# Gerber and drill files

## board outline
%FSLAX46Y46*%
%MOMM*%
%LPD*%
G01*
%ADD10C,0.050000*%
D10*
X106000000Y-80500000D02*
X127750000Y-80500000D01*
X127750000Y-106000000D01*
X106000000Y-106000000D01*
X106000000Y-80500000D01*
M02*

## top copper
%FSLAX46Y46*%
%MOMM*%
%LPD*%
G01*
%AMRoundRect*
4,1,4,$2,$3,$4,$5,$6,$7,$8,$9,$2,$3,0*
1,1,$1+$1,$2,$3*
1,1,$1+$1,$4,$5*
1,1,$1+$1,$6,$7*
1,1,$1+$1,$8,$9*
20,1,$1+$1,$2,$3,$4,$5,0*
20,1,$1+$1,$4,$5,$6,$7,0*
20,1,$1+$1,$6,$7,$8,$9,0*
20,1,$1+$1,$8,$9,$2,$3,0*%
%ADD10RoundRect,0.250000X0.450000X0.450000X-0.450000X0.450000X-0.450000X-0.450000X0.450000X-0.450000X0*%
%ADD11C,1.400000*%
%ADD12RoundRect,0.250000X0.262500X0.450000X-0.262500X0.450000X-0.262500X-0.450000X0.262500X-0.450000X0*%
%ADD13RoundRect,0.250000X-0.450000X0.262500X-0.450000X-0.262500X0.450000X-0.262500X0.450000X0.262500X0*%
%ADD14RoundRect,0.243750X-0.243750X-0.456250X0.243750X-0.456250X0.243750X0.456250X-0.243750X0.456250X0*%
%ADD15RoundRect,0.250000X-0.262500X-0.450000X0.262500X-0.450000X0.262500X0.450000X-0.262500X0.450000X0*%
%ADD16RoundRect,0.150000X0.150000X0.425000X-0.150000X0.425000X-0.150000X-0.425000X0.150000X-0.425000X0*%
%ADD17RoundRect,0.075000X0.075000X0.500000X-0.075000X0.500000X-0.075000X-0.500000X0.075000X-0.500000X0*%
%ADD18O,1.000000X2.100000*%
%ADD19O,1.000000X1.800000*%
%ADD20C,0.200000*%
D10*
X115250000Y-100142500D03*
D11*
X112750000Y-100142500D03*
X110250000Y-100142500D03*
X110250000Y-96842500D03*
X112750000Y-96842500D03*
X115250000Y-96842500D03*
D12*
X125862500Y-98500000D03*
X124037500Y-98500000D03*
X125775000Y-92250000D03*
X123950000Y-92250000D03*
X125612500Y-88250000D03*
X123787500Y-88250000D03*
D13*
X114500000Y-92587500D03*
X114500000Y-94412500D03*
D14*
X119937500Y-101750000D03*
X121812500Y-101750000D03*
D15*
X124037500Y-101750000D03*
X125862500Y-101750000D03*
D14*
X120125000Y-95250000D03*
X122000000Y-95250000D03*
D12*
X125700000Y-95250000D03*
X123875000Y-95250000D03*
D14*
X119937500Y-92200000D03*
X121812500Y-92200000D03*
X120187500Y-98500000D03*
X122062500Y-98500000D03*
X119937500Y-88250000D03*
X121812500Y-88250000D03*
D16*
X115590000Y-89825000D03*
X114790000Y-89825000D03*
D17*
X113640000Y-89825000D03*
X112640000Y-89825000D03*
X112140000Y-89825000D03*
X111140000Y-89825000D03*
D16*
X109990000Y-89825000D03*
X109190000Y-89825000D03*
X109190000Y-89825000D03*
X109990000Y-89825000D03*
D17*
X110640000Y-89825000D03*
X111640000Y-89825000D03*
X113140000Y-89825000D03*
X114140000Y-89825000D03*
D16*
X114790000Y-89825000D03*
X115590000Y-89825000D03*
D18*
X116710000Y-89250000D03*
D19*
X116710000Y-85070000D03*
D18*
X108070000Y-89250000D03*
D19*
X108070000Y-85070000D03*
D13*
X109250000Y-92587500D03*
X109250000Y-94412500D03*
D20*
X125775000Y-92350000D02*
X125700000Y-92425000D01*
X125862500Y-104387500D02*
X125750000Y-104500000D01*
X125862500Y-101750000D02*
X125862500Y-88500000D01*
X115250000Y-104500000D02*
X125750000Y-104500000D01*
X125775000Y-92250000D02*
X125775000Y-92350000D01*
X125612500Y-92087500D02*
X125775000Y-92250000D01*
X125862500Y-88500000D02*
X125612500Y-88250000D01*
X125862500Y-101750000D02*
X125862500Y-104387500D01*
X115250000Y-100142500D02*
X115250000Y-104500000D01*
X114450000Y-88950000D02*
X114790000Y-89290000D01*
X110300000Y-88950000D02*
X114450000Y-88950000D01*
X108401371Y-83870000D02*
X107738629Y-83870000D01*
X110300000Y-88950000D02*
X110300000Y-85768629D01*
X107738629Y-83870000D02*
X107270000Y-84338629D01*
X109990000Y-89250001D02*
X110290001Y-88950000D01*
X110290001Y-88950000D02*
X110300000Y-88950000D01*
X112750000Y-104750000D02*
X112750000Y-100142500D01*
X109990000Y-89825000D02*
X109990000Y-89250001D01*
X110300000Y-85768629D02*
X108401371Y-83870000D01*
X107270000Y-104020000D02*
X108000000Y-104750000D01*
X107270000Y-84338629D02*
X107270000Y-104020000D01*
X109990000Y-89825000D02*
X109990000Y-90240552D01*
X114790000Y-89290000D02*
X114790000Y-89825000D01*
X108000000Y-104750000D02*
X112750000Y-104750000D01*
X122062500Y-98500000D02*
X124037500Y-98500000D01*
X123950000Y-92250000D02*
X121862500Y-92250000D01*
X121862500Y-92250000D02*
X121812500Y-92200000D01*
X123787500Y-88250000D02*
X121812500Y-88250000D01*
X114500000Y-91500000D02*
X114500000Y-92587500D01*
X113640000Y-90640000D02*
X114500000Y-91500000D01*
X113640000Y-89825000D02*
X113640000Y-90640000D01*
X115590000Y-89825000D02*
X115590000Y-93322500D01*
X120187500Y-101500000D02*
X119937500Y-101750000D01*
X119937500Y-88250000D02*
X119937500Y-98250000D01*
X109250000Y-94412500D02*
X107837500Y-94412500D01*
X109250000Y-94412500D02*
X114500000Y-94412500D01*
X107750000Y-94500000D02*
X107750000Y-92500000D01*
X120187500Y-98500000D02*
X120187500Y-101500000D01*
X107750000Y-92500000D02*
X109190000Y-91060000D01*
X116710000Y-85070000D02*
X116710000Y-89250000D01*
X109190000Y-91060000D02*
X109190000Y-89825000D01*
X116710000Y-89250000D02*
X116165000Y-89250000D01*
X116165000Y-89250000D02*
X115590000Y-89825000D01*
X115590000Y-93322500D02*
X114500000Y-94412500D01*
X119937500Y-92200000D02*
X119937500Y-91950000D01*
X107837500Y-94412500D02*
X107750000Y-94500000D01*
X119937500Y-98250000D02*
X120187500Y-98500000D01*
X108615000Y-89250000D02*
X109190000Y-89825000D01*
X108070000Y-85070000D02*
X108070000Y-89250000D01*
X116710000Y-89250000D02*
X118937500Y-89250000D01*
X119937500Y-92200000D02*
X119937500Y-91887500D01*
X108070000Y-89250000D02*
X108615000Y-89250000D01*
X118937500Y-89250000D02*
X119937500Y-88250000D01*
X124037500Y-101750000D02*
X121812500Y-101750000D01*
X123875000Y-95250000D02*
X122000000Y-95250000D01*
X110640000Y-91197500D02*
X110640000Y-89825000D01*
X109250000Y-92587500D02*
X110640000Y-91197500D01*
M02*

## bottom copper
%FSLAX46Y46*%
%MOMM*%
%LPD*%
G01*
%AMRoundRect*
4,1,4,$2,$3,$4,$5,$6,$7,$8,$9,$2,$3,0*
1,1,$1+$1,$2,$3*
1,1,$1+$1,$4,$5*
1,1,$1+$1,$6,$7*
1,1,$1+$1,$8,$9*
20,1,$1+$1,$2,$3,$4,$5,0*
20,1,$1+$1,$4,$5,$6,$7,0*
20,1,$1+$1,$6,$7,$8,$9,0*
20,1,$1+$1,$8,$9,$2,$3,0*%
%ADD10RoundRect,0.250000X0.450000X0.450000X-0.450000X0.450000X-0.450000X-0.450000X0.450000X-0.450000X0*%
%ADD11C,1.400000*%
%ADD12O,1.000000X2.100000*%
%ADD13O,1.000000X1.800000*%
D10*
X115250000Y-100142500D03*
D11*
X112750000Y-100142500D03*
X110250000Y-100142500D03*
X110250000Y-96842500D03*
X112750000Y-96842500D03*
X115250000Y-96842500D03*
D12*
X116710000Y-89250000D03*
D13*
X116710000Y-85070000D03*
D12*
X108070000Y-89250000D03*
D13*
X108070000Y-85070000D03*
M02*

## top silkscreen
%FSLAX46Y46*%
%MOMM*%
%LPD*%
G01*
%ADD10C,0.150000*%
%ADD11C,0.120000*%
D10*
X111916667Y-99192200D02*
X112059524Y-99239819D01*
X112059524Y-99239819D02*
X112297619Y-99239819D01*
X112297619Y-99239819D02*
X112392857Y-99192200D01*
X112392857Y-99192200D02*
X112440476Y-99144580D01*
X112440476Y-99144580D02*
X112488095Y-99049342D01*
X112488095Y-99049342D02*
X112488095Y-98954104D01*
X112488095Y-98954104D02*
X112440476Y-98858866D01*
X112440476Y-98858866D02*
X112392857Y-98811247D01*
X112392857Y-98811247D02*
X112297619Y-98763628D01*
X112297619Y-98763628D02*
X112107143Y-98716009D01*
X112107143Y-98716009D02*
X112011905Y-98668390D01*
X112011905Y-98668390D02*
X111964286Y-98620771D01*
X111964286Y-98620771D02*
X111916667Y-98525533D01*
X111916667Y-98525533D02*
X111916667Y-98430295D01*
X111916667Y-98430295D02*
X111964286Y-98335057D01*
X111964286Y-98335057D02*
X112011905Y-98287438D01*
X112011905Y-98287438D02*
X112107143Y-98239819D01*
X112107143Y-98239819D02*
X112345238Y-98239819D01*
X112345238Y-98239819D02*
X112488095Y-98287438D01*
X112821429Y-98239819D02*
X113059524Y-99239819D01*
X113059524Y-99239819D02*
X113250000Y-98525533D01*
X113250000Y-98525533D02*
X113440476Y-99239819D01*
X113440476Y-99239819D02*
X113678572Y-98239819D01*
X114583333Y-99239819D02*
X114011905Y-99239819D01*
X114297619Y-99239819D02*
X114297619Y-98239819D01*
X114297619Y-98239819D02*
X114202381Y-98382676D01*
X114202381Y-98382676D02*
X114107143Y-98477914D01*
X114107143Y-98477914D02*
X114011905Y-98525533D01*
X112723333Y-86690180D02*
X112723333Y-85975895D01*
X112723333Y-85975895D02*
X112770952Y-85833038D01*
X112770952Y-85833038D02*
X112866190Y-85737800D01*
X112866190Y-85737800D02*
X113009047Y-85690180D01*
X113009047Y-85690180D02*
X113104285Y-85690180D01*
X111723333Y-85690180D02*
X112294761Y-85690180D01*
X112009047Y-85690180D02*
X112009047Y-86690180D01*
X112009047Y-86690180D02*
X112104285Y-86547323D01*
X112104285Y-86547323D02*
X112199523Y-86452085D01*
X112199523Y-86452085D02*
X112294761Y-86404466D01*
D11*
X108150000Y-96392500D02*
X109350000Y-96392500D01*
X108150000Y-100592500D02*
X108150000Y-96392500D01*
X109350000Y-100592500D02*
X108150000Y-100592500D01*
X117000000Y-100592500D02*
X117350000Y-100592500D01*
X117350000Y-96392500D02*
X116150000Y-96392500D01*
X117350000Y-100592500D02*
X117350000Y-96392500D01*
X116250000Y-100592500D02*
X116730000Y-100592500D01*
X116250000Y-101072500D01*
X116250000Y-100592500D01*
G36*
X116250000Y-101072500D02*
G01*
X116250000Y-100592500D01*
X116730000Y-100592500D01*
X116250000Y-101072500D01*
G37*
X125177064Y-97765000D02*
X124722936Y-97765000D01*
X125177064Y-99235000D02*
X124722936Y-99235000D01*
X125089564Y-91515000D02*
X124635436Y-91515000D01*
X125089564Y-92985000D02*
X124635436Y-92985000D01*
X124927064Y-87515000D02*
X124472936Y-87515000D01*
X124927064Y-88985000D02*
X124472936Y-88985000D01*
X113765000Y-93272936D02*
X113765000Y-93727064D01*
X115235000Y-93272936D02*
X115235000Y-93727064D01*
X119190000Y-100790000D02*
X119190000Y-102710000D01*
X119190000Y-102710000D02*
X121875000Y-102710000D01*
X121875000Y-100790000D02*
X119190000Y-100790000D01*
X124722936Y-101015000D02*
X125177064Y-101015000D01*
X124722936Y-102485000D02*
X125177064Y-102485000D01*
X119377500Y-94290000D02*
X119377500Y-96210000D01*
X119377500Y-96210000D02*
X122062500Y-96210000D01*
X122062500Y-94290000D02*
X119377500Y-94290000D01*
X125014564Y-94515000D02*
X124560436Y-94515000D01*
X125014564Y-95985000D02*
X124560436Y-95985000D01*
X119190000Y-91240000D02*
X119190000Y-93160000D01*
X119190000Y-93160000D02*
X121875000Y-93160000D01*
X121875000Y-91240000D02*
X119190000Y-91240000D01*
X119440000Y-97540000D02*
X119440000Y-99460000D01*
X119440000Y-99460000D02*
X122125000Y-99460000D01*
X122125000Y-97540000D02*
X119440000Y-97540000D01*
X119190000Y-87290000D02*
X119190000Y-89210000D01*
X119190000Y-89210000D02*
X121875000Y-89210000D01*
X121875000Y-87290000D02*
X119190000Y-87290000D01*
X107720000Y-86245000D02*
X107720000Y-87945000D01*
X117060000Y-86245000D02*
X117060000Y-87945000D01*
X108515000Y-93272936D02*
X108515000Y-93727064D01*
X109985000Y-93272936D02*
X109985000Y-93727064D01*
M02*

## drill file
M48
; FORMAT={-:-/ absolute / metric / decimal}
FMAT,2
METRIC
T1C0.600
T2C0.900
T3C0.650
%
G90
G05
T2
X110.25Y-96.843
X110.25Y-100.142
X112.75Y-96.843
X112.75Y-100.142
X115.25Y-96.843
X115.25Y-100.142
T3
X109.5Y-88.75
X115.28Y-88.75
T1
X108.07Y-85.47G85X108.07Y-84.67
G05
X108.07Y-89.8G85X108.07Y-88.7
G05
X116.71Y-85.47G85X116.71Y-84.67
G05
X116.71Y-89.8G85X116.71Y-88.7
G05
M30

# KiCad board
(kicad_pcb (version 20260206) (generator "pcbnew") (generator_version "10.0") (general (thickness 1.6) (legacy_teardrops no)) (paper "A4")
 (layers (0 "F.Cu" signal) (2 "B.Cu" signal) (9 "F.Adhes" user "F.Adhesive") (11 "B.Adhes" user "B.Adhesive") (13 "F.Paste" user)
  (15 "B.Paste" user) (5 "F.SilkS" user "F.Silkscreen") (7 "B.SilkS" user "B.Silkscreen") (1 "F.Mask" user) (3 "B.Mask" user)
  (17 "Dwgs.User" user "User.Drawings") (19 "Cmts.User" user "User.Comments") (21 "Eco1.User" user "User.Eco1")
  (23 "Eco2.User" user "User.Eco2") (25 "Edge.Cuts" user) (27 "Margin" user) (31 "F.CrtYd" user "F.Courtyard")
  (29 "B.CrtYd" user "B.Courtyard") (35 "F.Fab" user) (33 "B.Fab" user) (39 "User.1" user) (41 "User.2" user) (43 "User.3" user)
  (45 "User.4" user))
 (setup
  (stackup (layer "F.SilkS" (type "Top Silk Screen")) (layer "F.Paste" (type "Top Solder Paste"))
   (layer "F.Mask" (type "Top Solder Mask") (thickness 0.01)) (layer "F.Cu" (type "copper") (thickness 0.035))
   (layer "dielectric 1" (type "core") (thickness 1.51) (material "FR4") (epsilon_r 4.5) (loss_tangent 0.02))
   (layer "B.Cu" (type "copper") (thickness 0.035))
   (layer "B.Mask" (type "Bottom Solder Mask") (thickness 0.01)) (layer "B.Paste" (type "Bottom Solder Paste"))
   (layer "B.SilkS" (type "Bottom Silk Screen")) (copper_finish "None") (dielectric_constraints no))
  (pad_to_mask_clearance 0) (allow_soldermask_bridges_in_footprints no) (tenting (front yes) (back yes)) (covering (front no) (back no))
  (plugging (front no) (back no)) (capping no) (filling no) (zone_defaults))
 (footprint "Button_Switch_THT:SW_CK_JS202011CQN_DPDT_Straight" (layer "F.Cu") (at 115.25 100.1425 180)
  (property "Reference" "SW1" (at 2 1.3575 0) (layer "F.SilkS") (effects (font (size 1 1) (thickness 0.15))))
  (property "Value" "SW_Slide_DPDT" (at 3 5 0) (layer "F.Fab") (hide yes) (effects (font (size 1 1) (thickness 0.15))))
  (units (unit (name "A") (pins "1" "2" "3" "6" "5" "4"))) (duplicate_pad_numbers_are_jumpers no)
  (fp_line (start 7.1 3.75) (end 5.9 3.75) (stroke (width 0.12) (type solid)) (layer "F.SilkS"))
  (fp_line (start 7.1 -0.45) (end 7.1 3.75) (stroke (width 0.12) (type solid)) (layer "F.SilkS"))
  (fp_line (start 5.9 -0.45) (end 7.1 -0.45) (stroke (width 0.12) (type solid)) (layer "F.SilkS"))
  (fp_line (start -1.75 -0.45) (end -2.1 -0.45) (stroke (width 0.12) (type solid)) (layer "F.SilkS"))
  (fp_line (start -2.1 3.75) (end -0.9 3.75) (stroke (width 0.12) (type solid)) (layer "F.SilkS"))
  (fp_line (start -2.1 -0.45) (end -2.1 3.75) (stroke (width 0.12) (type solid)) (layer "F.SilkS"))
  (fp_poly (pts (xy -1 -0.45) (xy -1.48 -0.45) (xy -1 -0.93) (xy -1 -0.45)) (stroke (width 0.12) (type solid)) (fill yes) (layer "F.SilkS"))
  (pad "1" thru_hole roundrect (at 0 0 180) (size 1.4 1.4) (drill 0.9) (layers "*.Cu" "*.Mask") (remove_unused_layers no)
   (roundrect_rratio 0.1785714286) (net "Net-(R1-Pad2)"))
  (pad "2" thru_hole circle (at 2.5 0 180) (size 1.4 1.4) (drill 0.9) (layers "*.Cu" "*.Mask") (remove_unused_layers no)
   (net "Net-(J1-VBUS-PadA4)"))
  (pad "3" thru_hole circle (at 5 0 180) (size 1.4 1.4) (drill 0.9) (layers "*.Cu" "*.Mask") (remove_unused_layers no)
   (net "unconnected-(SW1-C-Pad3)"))
  (pad "4" thru_hole circle (at 5 3.3 180) (size 1.4 1.4) (drill 0.9) (layers "*.Cu" "*.Mask") (remove_unused_layers no)
   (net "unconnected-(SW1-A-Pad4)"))
  (pad "5" thru_hole circle (at 2.5 3.3 180) (size 1.4 1.4) (drill 0.9) (layers "*.Cu" "*.Mask") (remove_unused_layers no)
   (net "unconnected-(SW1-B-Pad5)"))
  (pad "6" thru_hole circle (at 0 3.3 180) (size 1.4 1.4) (drill 0.9) (layers "*.Cu" "*.Mask") (remove_unused_layers no)
   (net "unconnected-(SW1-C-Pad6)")))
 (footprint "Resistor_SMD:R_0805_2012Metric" (layer "F.Cu") (at 124.95 98.5 180)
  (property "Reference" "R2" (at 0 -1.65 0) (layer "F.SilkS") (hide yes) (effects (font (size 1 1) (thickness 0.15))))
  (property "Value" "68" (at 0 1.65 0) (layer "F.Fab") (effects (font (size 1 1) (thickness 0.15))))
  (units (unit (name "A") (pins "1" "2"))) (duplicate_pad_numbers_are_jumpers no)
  (fp_line (start -0.227064 0.735) (end 0.227064 0.735) (stroke (width 0.12) (type solid)) (layer "F.SilkS"))
  (fp_line (start -0.227064 -0.735) (end 0.227064 -0.735) (stroke (width 0.12) (type solid)) (layer "F.SilkS"))
  (pad "1" smd roundrect (at -0.9125 0 180) (size 1.025 1.4) (layers "F.Cu" "F.Mask" "F.Paste") (roundrect_rratio 0.243902)
   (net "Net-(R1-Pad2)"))
  (pad "2" smd roundrect (at 0.9125 0 180) (size 1.025 1.4) (layers "F.Cu" "F.Mask" "F.Paste") (roundrect_rratio 0.243902)
   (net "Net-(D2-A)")))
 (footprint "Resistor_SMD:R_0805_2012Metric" (layer "F.Cu") (at 124.8625 92.25 180)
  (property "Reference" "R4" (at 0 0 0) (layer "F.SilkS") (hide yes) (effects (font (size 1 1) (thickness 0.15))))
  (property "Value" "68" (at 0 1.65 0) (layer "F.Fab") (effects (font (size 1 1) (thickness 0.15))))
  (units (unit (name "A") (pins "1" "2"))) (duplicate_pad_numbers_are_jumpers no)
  (fp_line (start -0.227064 0.735) (end 0.227064 0.735) (stroke (width 0.12) (type solid)) (layer "F.SilkS"))
  (fp_line (start -0.227064 -0.735) (end 0.227064 -0.735) (stroke (width 0.12) (type solid)) (layer "F.SilkS"))
  (pad "1" smd roundrect (at -0.9125 0 180) (size 1.025 1.4) (layers "F.Cu" "F.Mask" "F.Paste") (roundrect_rratio 0.243902)
   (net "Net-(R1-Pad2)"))
  (pad "2" smd roundrect (at 0.9125 0 180) (size 1.025 1.4) (layers "F.Cu" "F.Mask" "F.Paste") (roundrect_rratio 0.243902)
   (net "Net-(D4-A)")))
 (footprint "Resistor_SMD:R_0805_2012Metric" (layer "F.Cu") (at 124.7 88.25 180)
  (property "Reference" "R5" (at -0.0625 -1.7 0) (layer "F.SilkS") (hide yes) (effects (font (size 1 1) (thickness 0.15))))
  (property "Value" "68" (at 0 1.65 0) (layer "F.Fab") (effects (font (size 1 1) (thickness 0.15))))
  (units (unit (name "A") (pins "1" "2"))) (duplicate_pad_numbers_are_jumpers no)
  (fp_line (start -0.227064 0.735) (end 0.227064 0.735) (stroke (width 0.12) (type solid)) (layer "F.SilkS"))
  (fp_line (start -0.227064 -0.735) (end 0.227064 -0.735) (stroke (width 0.12) (type solid)) (layer "F.SilkS"))
  (pad "1" smd roundrect (at -0.9125 0 180) (size 1.025 1.4) (layers "F.Cu" "F.Mask" "F.Paste") (roundrect_rratio 0.243902)
   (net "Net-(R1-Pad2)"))
  (pad "2" smd roundrect (at 0.9125 0 180) (size 1.025 1.4) (layers "F.Cu" "F.Mask" "F.Paste") (roundrect_rratio 0.243902)
   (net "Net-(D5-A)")))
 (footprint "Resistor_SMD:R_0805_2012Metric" (layer "F.Cu") (at 114.5 93.5 -90)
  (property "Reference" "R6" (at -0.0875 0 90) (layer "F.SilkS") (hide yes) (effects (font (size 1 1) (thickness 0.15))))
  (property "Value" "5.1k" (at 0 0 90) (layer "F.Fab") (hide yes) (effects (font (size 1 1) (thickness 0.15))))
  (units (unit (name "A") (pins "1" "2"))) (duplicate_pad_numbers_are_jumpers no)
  (fp_line (start -0.227064 0.735) (end 0.227064 0.735) (stroke (width 0.12) (type solid)) (layer "F.SilkS"))
  (fp_line (start -0.227064 -0.735) (end 0.227064 -0.735) (stroke (width 0.12) (type solid)) (layer "F.SilkS"))
  (pad "1" smd roundrect (at -0.9125 0 270) (size 1.025 1.4) (layers "F.Cu" "F.Mask" "F.Paste") (roundrect_rratio 0.243902)
   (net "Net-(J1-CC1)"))
  (pad "2" smd roundrect (at 0.9125 0 270) (size 1.025 1.4) (layers "F.Cu" "F.Mask" "F.Paste") (roundrect_rratio 0.243902)
   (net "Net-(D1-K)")))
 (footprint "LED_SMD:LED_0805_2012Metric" (layer "F.Cu") (at 120.875 101.75)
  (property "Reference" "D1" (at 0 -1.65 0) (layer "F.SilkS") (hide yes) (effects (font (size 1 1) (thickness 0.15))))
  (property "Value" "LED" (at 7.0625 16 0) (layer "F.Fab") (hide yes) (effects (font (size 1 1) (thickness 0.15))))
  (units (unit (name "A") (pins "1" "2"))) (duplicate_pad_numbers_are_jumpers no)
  (fp_line (start -1.685 -0.96) (end -1.685 0.96) (stroke (width 0.12) (type solid)) (layer "F.SilkS"))
  (fp_line (start -1.685 0.96) (end 1 0.96) (stroke (width 0.12) (type solid)) (layer "F.SilkS"))
  (fp_line (start 1 -0.96) (end -1.685 -0.96) (stroke (width 0.12) (type solid)) (layer "F.SilkS"))
  (pad "1" smd roundrect (at -0.9375 0) (size 0.975 1.4) (layers "F.Cu" "F.Mask" "F.Paste") (roundrect_rratio 0.25) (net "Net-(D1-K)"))
  (pad "2" smd roundrect (at 0.9375 0) (size 0.975 1.4) (layers "F.Cu" "F.Mask" "F.Paste") (roundrect_rratio 0.25) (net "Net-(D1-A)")))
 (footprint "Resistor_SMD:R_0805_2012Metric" (layer "F.Cu") (at 124.95 101.75)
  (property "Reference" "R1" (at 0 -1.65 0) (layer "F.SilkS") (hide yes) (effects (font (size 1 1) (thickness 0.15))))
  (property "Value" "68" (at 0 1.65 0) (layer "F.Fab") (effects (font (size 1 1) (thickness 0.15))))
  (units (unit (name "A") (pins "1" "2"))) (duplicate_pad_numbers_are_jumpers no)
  (fp_line (start -0.227064 -0.735) (end 0.227064 -0.735) (stroke (width 0.12) (type solid)) (layer "F.SilkS"))
  (fp_line (start -0.227064 0.735) (end 0.227064 0.735) (stroke (width 0.12) (type solid)) (layer "F.SilkS"))
  (pad "1" smd roundrect (at -0.9125 0) (size 1.025 1.4) (layers "F.Cu" "F.Mask" "F.Paste") (roundrect_rratio 0.243902) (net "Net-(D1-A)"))
  (pad "2" smd roundrect (at 0.9125 0) (size 1.025 1.4) (layers "F.Cu" "F.Mask" "F.Paste") (roundrect_rratio 0.243902) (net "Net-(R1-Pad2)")))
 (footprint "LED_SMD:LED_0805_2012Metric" (layer "F.Cu") (at 121.0625 95.25)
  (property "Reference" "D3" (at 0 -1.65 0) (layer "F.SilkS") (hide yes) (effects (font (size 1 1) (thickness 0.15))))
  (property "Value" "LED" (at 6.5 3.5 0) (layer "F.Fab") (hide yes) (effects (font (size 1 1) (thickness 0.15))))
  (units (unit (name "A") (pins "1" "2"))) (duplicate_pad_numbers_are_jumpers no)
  (fp_line (start -1.685 -0.96) (end -1.685 0.96) (stroke (width 0.12) (type solid)) (layer "F.SilkS"))
  (fp_line (start -1.685 0.96) (end 1 0.96) (stroke (width 0.12) (type solid)) (layer "F.SilkS"))
  (fp_line (start 1 -0.96) (end -1.685 -0.96) (stroke (width 0.12) (type solid)) (layer "F.SilkS"))
  (pad "1" smd roundrect (at -0.9375 0) (size 0.975 1.4) (layers "F.Cu" "F.Mask" "F.Paste") (roundrect_rratio 0.25) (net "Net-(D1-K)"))
  (pad "2" smd roundrect (at 0.9375 0) (size 0.975 1.4) (layers "F.Cu" "F.Mask" "F.Paste") (roundrect_rratio 0.25) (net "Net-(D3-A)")))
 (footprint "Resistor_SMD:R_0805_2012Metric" (layer "F.Cu") (at 124.7875 95.25 180)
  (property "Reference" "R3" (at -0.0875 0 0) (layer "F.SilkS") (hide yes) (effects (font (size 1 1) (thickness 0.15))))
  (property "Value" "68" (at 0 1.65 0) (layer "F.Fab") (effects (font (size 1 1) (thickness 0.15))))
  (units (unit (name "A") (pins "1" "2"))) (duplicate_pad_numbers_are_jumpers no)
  (fp_line (start -0.227064 0.735) (end 0.227064 0.735) (stroke (width 0.12) (type solid)) (layer "F.SilkS"))
  (fp_line (start -0.227064 -0.735) (end 0.227064 -0.735) (stroke (width 0.12) (type solid)) (layer "F.SilkS"))
  (pad "1" smd roundrect (at -0.9125 0 180) (size 1.025 1.4) (layers "F.Cu" "F.Mask" "F.Paste") (roundrect_rratio 0.243902)
   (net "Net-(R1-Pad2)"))
  (pad "2" smd roundrect (at 0.9125 0 180) (size 1.025 1.4) (layers "F.Cu" "F.Mask" "F.Paste") (roundrect_rratio 0.243902)
   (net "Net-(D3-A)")))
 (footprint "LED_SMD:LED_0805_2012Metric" (layer "F.Cu") (at 120.875 92.2)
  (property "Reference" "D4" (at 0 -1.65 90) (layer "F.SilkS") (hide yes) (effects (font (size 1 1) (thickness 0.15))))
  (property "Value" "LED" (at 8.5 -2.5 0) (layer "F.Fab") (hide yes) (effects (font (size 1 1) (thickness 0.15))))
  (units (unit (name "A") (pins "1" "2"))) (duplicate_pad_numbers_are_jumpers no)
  (fp_line (start -1.685 -0.96) (end -1.685 0.96) (stroke (width 0.12) (type solid)) (layer "F.SilkS"))
  (fp_line (start -1.685 0.96) (end 1 0.96) (stroke (width 0.12) (type solid)) (layer "F.SilkS"))
  (fp_line (start 1 -0.96) (end -1.685 -0.96) (stroke (width 0.12) (type solid)) (layer "F.SilkS"))
  (pad "1" smd roundrect (at -0.9375 0) (size 0.975 1.4) (layers "F.Cu" "F.Mask" "F.Paste") (roundrect_rratio 0.25) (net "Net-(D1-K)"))
  (pad "2" smd roundrect (at 0.9375 0) (size 0.975 1.4) (layers "F.Cu" "F.Mask" "F.Paste") (roundrect_rratio 0.25) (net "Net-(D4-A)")))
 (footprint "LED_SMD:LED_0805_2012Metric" (layer "F.Cu") (at 121.125 98.5)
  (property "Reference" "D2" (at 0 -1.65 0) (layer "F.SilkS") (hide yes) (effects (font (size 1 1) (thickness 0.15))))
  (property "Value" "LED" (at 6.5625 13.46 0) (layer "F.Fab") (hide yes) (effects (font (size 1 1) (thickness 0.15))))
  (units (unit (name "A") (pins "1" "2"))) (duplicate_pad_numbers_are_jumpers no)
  (fp_line (start -1.685 -0.96) (end -1.685 0.96) (stroke (width 0.12) (type solid)) (layer "F.SilkS"))
  (fp_line (start -1.685 0.96) (end 1 0.96) (stroke (width 0.12) (type solid)) (layer "F.SilkS"))
  (fp_line (start 1 -0.96) (end -1.685 -0.96) (stroke (width 0.12) (type solid)) (layer "F.SilkS"))
  (pad "1" smd roundrect (at -0.9375 0) (size 0.975 1.4) (layers "F.Cu" "F.Mask" "F.Paste") (roundrect_rratio 0.25) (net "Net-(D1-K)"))
  (pad "2" smd roundrect (at 0.9375 0) (size 0.975 1.4) (layers "F.Cu" "F.Mask" "F.Paste") (roundrect_rratio 0.25) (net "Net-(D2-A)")))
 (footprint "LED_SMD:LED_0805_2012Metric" (layer "F.Cu") (at 120.875 88.25)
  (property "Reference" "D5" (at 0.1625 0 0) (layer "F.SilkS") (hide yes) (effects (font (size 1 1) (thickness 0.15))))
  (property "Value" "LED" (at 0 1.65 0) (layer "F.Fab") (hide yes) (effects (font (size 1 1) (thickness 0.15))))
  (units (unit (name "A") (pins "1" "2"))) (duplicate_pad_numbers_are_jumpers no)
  (fp_line (start -1.685 -0.96) (end -1.685 0.96) (stroke (width 0.12) (type solid)) (layer "F.SilkS"))
  (fp_line (start -1.685 0.96) (end 1 0.96) (stroke (width 0.12) (type solid)) (layer "F.SilkS"))
  (fp_line (start 1 -0.96) (end -1.685 -0.96) (stroke (width 0.12) (type solid)) (layer "F.SilkS"))
  (pad "1" smd roundrect (at -0.9375 0) (size 0.975 1.4) (layers "F.Cu" "F.Mask" "F.Paste") (roundrect_rratio 0.25) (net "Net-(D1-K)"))
  (pad "2" smd roundrect (at 0.9375 0) (size 0.975 1.4) (layers "F.Cu" "F.Mask" "F.Paste") (roundrect_rratio 0.25) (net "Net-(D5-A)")))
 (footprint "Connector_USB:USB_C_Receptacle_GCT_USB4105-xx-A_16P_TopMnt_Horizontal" (layer "F.Cu") (at 112.39 86.145 180)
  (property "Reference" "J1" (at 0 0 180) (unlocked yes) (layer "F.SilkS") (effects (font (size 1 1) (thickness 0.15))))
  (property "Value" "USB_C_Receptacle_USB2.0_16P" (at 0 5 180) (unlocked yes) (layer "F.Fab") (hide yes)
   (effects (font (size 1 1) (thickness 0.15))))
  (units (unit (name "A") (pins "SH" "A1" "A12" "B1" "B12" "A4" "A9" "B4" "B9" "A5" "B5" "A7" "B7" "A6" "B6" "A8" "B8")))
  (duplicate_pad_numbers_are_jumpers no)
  (fp_line (start 4.67 -0.1) (end 4.67 -1.8) (stroke (width 0.12) (type solid)) (layer "F.SilkS"))
  (fp_line (start -4.67 -0.1) (end -4.67 -1.8) (stroke (width 0.12) (type solid)) (layer "F.SilkS"))
  (pad "" np_thru_hole circle (at -2.89 -2.605 180) (size 0.65 0.65) (drill 0.65) (layers "*.Cu" "*.Mask"))
  (pad "" np_thru_hole circle (at 2.89 -2.605 180) (size 0.65 0.65) (drill 0.65) (layers "*.Cu" "*.Mask"))
  (pad "A1" smd roundrect (at -3.2 -3.68 180) (size 0.6 1.15) (layers "F.Cu" "F.Mask" "F.Paste") (roundrect_rratio 0.25) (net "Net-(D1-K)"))
  (pad "A4" smd roundrect (at -2.4 -3.68 180) (size 0.6 1.15) (layers "F.Cu" "F.Mask" "F.Paste") (roundrect_rratio 0.25)
   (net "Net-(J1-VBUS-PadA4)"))
  (pad "A5" smd roundrect (at -1.25 -3.68 180) (size 0.3 1.15) (layers "F.Cu" "F.Mask" "F.Paste") (roundrect_rratio 0.25)
   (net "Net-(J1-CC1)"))
  (pad "A6" smd roundrect (at -0.25 -3.68 180) (size 0.3 1.15) (layers "F.Cu" "F.Mask" "F.Paste") (roundrect_rratio 0.25)
   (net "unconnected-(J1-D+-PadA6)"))
  (pad "A7" smd roundrect (at 0.25 -3.68 180) (size 0.3 1.15) (layers "F.Cu" "F.Mask" "F.Paste") (roundrect_rratio 0.25)
   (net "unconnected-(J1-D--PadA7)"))
  (pad "A8" smd roundrect (at 1.25 -3.68 180) (size 0.3 1.15) (layers "F.Cu" "F.Mask" "F.Paste") (roundrect_rratio 0.25)
   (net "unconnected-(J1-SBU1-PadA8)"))
  (pad "A9" smd roundrect (at 2.4 -3.68 180) (size 0.6 1.15) (layers "F.Cu" "F.Mask" "F.Paste") (roundrect_rratio 0.25)
   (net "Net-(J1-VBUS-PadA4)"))
  (pad "A12" smd roundrect (at 3.2 -3.68 180) (size 0.6 1.15) (layers "F.Cu" "F.Mask" "F.Paste") (roundrect_rratio 0.25) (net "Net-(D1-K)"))
  (pad "B1" smd roundrect (at 3.2 -3.68 180) (size 0.6 1.15) (layers "F.Cu" "F.Mask" "F.Paste") (roundrect_rratio 0.25) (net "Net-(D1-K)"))
  (pad "B4" smd roundrect (at 2.4 -3.68 180) (size 0.6 1.15) (layers "F.Cu" "F.Mask" "F.Paste") (roundrect_rratio 0.25)
   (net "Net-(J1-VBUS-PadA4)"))
  (pad "B5" smd roundrect (at 1.75 -3.68 180) (size 0.3 1.15) (layers "F.Cu" "F.Mask" "F.Paste") (roundrect_rratio 0.25)
   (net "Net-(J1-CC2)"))
  (pad "B6" smd roundrect (at 0.75 -3.68 180) (size 0.3 1.15) (layers "F.Cu" "F.Mask" "F.Paste") (roundrect_rratio 0.25)
   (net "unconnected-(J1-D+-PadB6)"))
  (pad "B7" smd roundrect (at -0.75 -3.68 180) (size 0.3 1.15) (layers "F.Cu" "F.Mask" "F.Paste") (roundrect_rratio 0.25)
   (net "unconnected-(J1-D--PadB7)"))
  (pad "B8" smd roundrect (at -1.75 -3.68 180) (size 0.3 1.15) (layers "F.Cu" "F.Mask" "F.Paste") (roundrect_rratio 0.25)
   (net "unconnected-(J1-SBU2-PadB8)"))
  (pad "B9" smd roundrect (at -2.4 -3.68 180) (size 0.6 1.15) (layers "F.Cu" "F.Mask" "F.Paste") (roundrect_rratio 0.25)
   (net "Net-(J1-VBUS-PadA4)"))
  (pad "B12" smd roundrect (at -3.2 -3.68 180) (size 0.6 1.15) (layers "F.Cu" "F.Mask" "F.Paste") (roundrect_rratio 0.25) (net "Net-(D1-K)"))
  (pad "SH" thru_hole oval (at -4.32 -3.105 180) (size 1 2.1) (drill oval 0.6 1.7) (layers "*.Cu" "*.Mask" "F.Paste")
   (remove_unused_layers no) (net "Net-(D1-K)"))
  (pad "SH" thru_hole oval (at -4.32 1.075 180) (size 1 1.8) (drill oval 0.6 1.4) (layers "*.Cu" "*.Mask" "F.Paste")
   (remove_unused_layers no) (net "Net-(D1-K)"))
  (pad "SH" thru_hole oval (at 4.32 -3.105 180) (size 1 2.1) (drill oval 0.6 1.7) (layers "*.Cu" "*.Mask" "F.Paste")
   (remove_unused_layers no) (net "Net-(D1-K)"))
  (pad "SH" thru_hole oval (at 4.32 1.075 180) (size 1 1.8) (drill oval 0.6 1.4) (layers "*.Cu" "*.Mask" "F.Paste")
   (remove_unused_layers no) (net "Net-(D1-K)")))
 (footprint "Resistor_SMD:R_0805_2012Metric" (layer "F.Cu") (at 109.25 93.5 -90)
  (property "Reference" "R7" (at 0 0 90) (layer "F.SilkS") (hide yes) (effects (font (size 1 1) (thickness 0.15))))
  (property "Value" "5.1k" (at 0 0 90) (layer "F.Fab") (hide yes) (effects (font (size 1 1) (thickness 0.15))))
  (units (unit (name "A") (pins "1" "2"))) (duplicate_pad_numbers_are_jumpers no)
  (fp_line (start -0.227064 0.735) (end 0.227064 0.735) (stroke (width 0.12) (type solid)) (layer "F.SilkS"))
  (fp_line (start -0.227064 -0.735) (end 0.227064 -0.735) (stroke (width 0.12) (type solid)) (layer "F.SilkS"))
  (pad "1" smd roundrect (at -0.9125 0 270) (size 1.025 1.4) (layers "F.Cu" "F.Mask" "F.Paste") (roundrect_rratio 0.243902)
   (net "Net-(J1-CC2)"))
  (pad "2" smd roundrect (at 0.9125 0 270) (size 1.025 1.4) (layers "F.Cu" "F.Mask" "F.Paste") (roundrect_rratio 0.243902)
   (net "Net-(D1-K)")))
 (gr_rect (start 106 80.5) (end 127.75 106) (stroke (width 0.05) (type default)) (fill no) (layer "Edge.Cuts"))
 (segment (start 125.775 92.35) (end 125.7 92.425) (width 0.2) (layer "F.Cu") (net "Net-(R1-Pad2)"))
 (segment (start 125.8625 104.3875) (end 125.75 104.5) (width 0.2) (layer "F.Cu") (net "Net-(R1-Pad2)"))
 (segment (start 125.8625 101.75) (end 125.8625 88.5) (width 0.2) (layer "F.Cu") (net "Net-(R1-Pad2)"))
 (segment (start 115.25 104.5) (end 125.75 104.5) (width 0.2) (layer "F.Cu") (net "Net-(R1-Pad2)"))
 (segment (start 125.775 92.25) (end 125.775 92.35) (width 0.2) (layer "F.Cu") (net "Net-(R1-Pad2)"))
 (segment (start 125.6125 92.0875) (end 125.775 92.25) (width 0.2) (layer "F.Cu") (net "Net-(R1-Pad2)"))
 (segment (start 125.8625 88.5) (end 125.6125 88.25) (width 0.2) (layer "F.Cu") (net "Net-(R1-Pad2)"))
 (segment (start 125.8625 101.75) (end 125.8625 104.3875) (width 0.2) (layer "F.Cu") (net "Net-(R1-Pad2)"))
 (segment (start 115.25 100.1425) (end 115.25 104.5) (width 0.2) (layer "F.Cu") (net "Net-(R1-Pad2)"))
 (segment (start 114.45 88.95) (end 114.79 89.29) (width 0.2) (layer "F.Cu") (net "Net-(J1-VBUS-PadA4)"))
 (segment (start 110.3 88.95) (end 114.45 88.95) (width 0.2) (layer "F.Cu") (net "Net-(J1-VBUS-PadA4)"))
 (segment (start 108.401371 83.87) (end 107.738629 83.87) (width 0.2) (layer "F.Cu") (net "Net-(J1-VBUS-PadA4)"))
 (segment (start 110.3 88.95) (end 110.3 85.768629) (width 0.2) (layer "F.Cu") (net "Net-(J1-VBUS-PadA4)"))
 (segment (start 107.738629 83.87) (end 107.27 84.338629) (width 0.2) (layer "F.Cu") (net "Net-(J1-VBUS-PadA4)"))
 (segment (start 109.99 89.250001) (end 110.290001 88.95) (width 0.2) (layer "F.Cu") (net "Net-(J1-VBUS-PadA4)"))
 (segment (start 110.290001 88.95) (end 110.3 88.95) (width 0.2) (layer "F.Cu") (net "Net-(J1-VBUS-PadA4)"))
 (segment (start 112.75 104.75) (end 112.75 100.1425) (width 0.2) (layer "F.Cu") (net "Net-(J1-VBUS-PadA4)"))
 (segment (start 109.99 89.825) (end 109.99 89.250001) (width 0.2) (layer "F.Cu") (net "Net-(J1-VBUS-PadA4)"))
 (segment (start 110.3 85.768629) (end 108.401371 83.87) (width 0.2) (layer "F.Cu") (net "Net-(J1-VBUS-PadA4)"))
 (segment (start 107.27 104.02) (end 108 104.75) (width 0.2) (layer "F.Cu") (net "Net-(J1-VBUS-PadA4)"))
 (segment (start 107.27 84.338629) (end 107.27 104.02) (width 0.2) (layer "F.Cu") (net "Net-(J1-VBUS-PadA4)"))
 (segment (start 109.99 89.825) (end 109.99 90.240552) (width 0.2) (layer "F.Cu") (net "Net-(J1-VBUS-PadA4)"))
 (segment (start 114.79 89.29) (end 114.79 89.825) (width 0.2) (layer "F.Cu") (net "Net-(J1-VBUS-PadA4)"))
 (segment (start 108 104.75) (end 112.75 104.75) (width 0.2) (layer "F.Cu") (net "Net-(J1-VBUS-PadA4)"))
 (segment (start 122.0625 98.5) (end 124.0375 98.5) (width 0.2) (layer "F.Cu") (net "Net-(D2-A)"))
 (segment (start 123.95 92.25) (end 121.8625 92.25) (width 0.2) (layer "F.Cu") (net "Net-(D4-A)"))
 (segment (start 121.8625 92.25) (end 121.8125 92.2) (width 0.2) (layer "F.Cu") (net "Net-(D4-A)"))
 (segment (start 123.7875 88.25) (end 121.8125 88.25) (width 0.2) (layer "F.Cu") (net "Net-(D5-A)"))
 (segment (start 114.5 91.5) (end 114.5 92.5875) (width 0.2) (layer "F.Cu") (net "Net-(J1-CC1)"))
 (segment (start 113.64 90.64) (end 114.5 91.5) (width 0.2) (layer "F.Cu") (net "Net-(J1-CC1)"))
 (segment (start 113.64 89.825) (end 113.64 90.64) (width 0.2) (layer "F.Cu") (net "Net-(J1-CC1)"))
 (segment (start 115.59 89.825) (end 115.59 93.3225) (width 0.2) (layer "F.Cu") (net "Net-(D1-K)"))
 (segment (start 120.1875 101.5) (end 119.9375 101.75) (width 0.2) (layer "F.Cu") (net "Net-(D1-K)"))
 (segment (start 119.9375 88.25) (end 119.9375 98.25) (width 0.2) (layer "F.Cu") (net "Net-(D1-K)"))
 (segment (start 109.25 94.4125) (end 107.8375 94.4125) (width 0.2) (layer "F.Cu") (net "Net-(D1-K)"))
 (segment (start 109.25 94.4125) (end 114.5 94.4125) (width 0.2) (layer "F.Cu") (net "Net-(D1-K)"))
 (segment (start 107.75 94.5) (end 107.75 92.5) (width 0.2) (layer "F.Cu") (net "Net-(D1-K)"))
 (segment (start 120.1875 98.5) (end 120.1875 101.5) (width 0.2) (layer "F.Cu") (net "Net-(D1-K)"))
 (segment (start 107.75 92.5) (end 109.19 91.06) (width 0.2) (layer "F.Cu") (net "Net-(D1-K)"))
 (segment (start 116.71 85.07) (end 116.71 89.25) (width 0.2) (layer "F.Cu") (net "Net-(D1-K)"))
 (segment (start 109.19 91.06) (end 109.19 89.825) (width 0.2) (layer "F.Cu") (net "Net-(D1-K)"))
 (segment (start 116.71 89.25) (end 116.165 89.25) (width 0.2) (layer "F.Cu") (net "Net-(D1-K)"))
 (segment (start 116.165 89.25) (end 115.59 89.825) (width 0.2) (layer "F.Cu") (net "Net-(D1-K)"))
 (segment (start 115.59 93.3225) (end 114.5 94.4125) (width 0.2) (layer "F.Cu") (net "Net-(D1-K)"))
 (segment (start 119.9375 92.2) (end 119.9375 91.95) (width 0.2) (layer "F.Cu") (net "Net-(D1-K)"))
 (segment (start 107.8375 94.4125) (end 107.75 94.5) (width 0.2) (layer "F.Cu") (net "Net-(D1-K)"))
 (segment (start 119.9375 98.25) (end 120.1875 98.5) (width 0.2) (layer "F.Cu") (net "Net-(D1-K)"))
 (segment (start 108.615 89.25) (end 109.19 89.825) (width 0.2) (layer "F.Cu") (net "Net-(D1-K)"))
 (segment (start 108.07 85.07) (end 108.07 89.25) (width 0.2) (layer "F.Cu") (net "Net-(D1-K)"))
 (segment (start 116.71 89.25) (end 118.9375 89.25) (width 0.2) (layer "F.Cu") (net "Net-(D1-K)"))
 (segment (start 119.9375 92.2) (end 119.9375 91.8875) (width 0.2) (layer "F.Cu") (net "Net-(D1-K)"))
 (segment (start 108.07 89.25) (end 108.615 89.25) (width 0.2) (layer "F.Cu") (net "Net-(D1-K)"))
 (segment (start 118.9375 89.25) (end 119.9375 88.25) (width 0.2) (layer "F.Cu") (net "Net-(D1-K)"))
 (segment (start 124.0375 101.75) (end 121.8125 101.75) (width 0.2) (layer "F.Cu") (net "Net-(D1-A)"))
 (segment (start 123.875 95.25) (end 122 95.25) (width 0.2) (layer "F.Cu") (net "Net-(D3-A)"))
 (segment (start 110.64 91.1975) (end 110.64 89.825) (width 0.2) (layer "F.Cu") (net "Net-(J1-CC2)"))
 (segment (start 109.25 92.5875) (end 110.64 91.1975) (width 0.2) (layer "F.Cu") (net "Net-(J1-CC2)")))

